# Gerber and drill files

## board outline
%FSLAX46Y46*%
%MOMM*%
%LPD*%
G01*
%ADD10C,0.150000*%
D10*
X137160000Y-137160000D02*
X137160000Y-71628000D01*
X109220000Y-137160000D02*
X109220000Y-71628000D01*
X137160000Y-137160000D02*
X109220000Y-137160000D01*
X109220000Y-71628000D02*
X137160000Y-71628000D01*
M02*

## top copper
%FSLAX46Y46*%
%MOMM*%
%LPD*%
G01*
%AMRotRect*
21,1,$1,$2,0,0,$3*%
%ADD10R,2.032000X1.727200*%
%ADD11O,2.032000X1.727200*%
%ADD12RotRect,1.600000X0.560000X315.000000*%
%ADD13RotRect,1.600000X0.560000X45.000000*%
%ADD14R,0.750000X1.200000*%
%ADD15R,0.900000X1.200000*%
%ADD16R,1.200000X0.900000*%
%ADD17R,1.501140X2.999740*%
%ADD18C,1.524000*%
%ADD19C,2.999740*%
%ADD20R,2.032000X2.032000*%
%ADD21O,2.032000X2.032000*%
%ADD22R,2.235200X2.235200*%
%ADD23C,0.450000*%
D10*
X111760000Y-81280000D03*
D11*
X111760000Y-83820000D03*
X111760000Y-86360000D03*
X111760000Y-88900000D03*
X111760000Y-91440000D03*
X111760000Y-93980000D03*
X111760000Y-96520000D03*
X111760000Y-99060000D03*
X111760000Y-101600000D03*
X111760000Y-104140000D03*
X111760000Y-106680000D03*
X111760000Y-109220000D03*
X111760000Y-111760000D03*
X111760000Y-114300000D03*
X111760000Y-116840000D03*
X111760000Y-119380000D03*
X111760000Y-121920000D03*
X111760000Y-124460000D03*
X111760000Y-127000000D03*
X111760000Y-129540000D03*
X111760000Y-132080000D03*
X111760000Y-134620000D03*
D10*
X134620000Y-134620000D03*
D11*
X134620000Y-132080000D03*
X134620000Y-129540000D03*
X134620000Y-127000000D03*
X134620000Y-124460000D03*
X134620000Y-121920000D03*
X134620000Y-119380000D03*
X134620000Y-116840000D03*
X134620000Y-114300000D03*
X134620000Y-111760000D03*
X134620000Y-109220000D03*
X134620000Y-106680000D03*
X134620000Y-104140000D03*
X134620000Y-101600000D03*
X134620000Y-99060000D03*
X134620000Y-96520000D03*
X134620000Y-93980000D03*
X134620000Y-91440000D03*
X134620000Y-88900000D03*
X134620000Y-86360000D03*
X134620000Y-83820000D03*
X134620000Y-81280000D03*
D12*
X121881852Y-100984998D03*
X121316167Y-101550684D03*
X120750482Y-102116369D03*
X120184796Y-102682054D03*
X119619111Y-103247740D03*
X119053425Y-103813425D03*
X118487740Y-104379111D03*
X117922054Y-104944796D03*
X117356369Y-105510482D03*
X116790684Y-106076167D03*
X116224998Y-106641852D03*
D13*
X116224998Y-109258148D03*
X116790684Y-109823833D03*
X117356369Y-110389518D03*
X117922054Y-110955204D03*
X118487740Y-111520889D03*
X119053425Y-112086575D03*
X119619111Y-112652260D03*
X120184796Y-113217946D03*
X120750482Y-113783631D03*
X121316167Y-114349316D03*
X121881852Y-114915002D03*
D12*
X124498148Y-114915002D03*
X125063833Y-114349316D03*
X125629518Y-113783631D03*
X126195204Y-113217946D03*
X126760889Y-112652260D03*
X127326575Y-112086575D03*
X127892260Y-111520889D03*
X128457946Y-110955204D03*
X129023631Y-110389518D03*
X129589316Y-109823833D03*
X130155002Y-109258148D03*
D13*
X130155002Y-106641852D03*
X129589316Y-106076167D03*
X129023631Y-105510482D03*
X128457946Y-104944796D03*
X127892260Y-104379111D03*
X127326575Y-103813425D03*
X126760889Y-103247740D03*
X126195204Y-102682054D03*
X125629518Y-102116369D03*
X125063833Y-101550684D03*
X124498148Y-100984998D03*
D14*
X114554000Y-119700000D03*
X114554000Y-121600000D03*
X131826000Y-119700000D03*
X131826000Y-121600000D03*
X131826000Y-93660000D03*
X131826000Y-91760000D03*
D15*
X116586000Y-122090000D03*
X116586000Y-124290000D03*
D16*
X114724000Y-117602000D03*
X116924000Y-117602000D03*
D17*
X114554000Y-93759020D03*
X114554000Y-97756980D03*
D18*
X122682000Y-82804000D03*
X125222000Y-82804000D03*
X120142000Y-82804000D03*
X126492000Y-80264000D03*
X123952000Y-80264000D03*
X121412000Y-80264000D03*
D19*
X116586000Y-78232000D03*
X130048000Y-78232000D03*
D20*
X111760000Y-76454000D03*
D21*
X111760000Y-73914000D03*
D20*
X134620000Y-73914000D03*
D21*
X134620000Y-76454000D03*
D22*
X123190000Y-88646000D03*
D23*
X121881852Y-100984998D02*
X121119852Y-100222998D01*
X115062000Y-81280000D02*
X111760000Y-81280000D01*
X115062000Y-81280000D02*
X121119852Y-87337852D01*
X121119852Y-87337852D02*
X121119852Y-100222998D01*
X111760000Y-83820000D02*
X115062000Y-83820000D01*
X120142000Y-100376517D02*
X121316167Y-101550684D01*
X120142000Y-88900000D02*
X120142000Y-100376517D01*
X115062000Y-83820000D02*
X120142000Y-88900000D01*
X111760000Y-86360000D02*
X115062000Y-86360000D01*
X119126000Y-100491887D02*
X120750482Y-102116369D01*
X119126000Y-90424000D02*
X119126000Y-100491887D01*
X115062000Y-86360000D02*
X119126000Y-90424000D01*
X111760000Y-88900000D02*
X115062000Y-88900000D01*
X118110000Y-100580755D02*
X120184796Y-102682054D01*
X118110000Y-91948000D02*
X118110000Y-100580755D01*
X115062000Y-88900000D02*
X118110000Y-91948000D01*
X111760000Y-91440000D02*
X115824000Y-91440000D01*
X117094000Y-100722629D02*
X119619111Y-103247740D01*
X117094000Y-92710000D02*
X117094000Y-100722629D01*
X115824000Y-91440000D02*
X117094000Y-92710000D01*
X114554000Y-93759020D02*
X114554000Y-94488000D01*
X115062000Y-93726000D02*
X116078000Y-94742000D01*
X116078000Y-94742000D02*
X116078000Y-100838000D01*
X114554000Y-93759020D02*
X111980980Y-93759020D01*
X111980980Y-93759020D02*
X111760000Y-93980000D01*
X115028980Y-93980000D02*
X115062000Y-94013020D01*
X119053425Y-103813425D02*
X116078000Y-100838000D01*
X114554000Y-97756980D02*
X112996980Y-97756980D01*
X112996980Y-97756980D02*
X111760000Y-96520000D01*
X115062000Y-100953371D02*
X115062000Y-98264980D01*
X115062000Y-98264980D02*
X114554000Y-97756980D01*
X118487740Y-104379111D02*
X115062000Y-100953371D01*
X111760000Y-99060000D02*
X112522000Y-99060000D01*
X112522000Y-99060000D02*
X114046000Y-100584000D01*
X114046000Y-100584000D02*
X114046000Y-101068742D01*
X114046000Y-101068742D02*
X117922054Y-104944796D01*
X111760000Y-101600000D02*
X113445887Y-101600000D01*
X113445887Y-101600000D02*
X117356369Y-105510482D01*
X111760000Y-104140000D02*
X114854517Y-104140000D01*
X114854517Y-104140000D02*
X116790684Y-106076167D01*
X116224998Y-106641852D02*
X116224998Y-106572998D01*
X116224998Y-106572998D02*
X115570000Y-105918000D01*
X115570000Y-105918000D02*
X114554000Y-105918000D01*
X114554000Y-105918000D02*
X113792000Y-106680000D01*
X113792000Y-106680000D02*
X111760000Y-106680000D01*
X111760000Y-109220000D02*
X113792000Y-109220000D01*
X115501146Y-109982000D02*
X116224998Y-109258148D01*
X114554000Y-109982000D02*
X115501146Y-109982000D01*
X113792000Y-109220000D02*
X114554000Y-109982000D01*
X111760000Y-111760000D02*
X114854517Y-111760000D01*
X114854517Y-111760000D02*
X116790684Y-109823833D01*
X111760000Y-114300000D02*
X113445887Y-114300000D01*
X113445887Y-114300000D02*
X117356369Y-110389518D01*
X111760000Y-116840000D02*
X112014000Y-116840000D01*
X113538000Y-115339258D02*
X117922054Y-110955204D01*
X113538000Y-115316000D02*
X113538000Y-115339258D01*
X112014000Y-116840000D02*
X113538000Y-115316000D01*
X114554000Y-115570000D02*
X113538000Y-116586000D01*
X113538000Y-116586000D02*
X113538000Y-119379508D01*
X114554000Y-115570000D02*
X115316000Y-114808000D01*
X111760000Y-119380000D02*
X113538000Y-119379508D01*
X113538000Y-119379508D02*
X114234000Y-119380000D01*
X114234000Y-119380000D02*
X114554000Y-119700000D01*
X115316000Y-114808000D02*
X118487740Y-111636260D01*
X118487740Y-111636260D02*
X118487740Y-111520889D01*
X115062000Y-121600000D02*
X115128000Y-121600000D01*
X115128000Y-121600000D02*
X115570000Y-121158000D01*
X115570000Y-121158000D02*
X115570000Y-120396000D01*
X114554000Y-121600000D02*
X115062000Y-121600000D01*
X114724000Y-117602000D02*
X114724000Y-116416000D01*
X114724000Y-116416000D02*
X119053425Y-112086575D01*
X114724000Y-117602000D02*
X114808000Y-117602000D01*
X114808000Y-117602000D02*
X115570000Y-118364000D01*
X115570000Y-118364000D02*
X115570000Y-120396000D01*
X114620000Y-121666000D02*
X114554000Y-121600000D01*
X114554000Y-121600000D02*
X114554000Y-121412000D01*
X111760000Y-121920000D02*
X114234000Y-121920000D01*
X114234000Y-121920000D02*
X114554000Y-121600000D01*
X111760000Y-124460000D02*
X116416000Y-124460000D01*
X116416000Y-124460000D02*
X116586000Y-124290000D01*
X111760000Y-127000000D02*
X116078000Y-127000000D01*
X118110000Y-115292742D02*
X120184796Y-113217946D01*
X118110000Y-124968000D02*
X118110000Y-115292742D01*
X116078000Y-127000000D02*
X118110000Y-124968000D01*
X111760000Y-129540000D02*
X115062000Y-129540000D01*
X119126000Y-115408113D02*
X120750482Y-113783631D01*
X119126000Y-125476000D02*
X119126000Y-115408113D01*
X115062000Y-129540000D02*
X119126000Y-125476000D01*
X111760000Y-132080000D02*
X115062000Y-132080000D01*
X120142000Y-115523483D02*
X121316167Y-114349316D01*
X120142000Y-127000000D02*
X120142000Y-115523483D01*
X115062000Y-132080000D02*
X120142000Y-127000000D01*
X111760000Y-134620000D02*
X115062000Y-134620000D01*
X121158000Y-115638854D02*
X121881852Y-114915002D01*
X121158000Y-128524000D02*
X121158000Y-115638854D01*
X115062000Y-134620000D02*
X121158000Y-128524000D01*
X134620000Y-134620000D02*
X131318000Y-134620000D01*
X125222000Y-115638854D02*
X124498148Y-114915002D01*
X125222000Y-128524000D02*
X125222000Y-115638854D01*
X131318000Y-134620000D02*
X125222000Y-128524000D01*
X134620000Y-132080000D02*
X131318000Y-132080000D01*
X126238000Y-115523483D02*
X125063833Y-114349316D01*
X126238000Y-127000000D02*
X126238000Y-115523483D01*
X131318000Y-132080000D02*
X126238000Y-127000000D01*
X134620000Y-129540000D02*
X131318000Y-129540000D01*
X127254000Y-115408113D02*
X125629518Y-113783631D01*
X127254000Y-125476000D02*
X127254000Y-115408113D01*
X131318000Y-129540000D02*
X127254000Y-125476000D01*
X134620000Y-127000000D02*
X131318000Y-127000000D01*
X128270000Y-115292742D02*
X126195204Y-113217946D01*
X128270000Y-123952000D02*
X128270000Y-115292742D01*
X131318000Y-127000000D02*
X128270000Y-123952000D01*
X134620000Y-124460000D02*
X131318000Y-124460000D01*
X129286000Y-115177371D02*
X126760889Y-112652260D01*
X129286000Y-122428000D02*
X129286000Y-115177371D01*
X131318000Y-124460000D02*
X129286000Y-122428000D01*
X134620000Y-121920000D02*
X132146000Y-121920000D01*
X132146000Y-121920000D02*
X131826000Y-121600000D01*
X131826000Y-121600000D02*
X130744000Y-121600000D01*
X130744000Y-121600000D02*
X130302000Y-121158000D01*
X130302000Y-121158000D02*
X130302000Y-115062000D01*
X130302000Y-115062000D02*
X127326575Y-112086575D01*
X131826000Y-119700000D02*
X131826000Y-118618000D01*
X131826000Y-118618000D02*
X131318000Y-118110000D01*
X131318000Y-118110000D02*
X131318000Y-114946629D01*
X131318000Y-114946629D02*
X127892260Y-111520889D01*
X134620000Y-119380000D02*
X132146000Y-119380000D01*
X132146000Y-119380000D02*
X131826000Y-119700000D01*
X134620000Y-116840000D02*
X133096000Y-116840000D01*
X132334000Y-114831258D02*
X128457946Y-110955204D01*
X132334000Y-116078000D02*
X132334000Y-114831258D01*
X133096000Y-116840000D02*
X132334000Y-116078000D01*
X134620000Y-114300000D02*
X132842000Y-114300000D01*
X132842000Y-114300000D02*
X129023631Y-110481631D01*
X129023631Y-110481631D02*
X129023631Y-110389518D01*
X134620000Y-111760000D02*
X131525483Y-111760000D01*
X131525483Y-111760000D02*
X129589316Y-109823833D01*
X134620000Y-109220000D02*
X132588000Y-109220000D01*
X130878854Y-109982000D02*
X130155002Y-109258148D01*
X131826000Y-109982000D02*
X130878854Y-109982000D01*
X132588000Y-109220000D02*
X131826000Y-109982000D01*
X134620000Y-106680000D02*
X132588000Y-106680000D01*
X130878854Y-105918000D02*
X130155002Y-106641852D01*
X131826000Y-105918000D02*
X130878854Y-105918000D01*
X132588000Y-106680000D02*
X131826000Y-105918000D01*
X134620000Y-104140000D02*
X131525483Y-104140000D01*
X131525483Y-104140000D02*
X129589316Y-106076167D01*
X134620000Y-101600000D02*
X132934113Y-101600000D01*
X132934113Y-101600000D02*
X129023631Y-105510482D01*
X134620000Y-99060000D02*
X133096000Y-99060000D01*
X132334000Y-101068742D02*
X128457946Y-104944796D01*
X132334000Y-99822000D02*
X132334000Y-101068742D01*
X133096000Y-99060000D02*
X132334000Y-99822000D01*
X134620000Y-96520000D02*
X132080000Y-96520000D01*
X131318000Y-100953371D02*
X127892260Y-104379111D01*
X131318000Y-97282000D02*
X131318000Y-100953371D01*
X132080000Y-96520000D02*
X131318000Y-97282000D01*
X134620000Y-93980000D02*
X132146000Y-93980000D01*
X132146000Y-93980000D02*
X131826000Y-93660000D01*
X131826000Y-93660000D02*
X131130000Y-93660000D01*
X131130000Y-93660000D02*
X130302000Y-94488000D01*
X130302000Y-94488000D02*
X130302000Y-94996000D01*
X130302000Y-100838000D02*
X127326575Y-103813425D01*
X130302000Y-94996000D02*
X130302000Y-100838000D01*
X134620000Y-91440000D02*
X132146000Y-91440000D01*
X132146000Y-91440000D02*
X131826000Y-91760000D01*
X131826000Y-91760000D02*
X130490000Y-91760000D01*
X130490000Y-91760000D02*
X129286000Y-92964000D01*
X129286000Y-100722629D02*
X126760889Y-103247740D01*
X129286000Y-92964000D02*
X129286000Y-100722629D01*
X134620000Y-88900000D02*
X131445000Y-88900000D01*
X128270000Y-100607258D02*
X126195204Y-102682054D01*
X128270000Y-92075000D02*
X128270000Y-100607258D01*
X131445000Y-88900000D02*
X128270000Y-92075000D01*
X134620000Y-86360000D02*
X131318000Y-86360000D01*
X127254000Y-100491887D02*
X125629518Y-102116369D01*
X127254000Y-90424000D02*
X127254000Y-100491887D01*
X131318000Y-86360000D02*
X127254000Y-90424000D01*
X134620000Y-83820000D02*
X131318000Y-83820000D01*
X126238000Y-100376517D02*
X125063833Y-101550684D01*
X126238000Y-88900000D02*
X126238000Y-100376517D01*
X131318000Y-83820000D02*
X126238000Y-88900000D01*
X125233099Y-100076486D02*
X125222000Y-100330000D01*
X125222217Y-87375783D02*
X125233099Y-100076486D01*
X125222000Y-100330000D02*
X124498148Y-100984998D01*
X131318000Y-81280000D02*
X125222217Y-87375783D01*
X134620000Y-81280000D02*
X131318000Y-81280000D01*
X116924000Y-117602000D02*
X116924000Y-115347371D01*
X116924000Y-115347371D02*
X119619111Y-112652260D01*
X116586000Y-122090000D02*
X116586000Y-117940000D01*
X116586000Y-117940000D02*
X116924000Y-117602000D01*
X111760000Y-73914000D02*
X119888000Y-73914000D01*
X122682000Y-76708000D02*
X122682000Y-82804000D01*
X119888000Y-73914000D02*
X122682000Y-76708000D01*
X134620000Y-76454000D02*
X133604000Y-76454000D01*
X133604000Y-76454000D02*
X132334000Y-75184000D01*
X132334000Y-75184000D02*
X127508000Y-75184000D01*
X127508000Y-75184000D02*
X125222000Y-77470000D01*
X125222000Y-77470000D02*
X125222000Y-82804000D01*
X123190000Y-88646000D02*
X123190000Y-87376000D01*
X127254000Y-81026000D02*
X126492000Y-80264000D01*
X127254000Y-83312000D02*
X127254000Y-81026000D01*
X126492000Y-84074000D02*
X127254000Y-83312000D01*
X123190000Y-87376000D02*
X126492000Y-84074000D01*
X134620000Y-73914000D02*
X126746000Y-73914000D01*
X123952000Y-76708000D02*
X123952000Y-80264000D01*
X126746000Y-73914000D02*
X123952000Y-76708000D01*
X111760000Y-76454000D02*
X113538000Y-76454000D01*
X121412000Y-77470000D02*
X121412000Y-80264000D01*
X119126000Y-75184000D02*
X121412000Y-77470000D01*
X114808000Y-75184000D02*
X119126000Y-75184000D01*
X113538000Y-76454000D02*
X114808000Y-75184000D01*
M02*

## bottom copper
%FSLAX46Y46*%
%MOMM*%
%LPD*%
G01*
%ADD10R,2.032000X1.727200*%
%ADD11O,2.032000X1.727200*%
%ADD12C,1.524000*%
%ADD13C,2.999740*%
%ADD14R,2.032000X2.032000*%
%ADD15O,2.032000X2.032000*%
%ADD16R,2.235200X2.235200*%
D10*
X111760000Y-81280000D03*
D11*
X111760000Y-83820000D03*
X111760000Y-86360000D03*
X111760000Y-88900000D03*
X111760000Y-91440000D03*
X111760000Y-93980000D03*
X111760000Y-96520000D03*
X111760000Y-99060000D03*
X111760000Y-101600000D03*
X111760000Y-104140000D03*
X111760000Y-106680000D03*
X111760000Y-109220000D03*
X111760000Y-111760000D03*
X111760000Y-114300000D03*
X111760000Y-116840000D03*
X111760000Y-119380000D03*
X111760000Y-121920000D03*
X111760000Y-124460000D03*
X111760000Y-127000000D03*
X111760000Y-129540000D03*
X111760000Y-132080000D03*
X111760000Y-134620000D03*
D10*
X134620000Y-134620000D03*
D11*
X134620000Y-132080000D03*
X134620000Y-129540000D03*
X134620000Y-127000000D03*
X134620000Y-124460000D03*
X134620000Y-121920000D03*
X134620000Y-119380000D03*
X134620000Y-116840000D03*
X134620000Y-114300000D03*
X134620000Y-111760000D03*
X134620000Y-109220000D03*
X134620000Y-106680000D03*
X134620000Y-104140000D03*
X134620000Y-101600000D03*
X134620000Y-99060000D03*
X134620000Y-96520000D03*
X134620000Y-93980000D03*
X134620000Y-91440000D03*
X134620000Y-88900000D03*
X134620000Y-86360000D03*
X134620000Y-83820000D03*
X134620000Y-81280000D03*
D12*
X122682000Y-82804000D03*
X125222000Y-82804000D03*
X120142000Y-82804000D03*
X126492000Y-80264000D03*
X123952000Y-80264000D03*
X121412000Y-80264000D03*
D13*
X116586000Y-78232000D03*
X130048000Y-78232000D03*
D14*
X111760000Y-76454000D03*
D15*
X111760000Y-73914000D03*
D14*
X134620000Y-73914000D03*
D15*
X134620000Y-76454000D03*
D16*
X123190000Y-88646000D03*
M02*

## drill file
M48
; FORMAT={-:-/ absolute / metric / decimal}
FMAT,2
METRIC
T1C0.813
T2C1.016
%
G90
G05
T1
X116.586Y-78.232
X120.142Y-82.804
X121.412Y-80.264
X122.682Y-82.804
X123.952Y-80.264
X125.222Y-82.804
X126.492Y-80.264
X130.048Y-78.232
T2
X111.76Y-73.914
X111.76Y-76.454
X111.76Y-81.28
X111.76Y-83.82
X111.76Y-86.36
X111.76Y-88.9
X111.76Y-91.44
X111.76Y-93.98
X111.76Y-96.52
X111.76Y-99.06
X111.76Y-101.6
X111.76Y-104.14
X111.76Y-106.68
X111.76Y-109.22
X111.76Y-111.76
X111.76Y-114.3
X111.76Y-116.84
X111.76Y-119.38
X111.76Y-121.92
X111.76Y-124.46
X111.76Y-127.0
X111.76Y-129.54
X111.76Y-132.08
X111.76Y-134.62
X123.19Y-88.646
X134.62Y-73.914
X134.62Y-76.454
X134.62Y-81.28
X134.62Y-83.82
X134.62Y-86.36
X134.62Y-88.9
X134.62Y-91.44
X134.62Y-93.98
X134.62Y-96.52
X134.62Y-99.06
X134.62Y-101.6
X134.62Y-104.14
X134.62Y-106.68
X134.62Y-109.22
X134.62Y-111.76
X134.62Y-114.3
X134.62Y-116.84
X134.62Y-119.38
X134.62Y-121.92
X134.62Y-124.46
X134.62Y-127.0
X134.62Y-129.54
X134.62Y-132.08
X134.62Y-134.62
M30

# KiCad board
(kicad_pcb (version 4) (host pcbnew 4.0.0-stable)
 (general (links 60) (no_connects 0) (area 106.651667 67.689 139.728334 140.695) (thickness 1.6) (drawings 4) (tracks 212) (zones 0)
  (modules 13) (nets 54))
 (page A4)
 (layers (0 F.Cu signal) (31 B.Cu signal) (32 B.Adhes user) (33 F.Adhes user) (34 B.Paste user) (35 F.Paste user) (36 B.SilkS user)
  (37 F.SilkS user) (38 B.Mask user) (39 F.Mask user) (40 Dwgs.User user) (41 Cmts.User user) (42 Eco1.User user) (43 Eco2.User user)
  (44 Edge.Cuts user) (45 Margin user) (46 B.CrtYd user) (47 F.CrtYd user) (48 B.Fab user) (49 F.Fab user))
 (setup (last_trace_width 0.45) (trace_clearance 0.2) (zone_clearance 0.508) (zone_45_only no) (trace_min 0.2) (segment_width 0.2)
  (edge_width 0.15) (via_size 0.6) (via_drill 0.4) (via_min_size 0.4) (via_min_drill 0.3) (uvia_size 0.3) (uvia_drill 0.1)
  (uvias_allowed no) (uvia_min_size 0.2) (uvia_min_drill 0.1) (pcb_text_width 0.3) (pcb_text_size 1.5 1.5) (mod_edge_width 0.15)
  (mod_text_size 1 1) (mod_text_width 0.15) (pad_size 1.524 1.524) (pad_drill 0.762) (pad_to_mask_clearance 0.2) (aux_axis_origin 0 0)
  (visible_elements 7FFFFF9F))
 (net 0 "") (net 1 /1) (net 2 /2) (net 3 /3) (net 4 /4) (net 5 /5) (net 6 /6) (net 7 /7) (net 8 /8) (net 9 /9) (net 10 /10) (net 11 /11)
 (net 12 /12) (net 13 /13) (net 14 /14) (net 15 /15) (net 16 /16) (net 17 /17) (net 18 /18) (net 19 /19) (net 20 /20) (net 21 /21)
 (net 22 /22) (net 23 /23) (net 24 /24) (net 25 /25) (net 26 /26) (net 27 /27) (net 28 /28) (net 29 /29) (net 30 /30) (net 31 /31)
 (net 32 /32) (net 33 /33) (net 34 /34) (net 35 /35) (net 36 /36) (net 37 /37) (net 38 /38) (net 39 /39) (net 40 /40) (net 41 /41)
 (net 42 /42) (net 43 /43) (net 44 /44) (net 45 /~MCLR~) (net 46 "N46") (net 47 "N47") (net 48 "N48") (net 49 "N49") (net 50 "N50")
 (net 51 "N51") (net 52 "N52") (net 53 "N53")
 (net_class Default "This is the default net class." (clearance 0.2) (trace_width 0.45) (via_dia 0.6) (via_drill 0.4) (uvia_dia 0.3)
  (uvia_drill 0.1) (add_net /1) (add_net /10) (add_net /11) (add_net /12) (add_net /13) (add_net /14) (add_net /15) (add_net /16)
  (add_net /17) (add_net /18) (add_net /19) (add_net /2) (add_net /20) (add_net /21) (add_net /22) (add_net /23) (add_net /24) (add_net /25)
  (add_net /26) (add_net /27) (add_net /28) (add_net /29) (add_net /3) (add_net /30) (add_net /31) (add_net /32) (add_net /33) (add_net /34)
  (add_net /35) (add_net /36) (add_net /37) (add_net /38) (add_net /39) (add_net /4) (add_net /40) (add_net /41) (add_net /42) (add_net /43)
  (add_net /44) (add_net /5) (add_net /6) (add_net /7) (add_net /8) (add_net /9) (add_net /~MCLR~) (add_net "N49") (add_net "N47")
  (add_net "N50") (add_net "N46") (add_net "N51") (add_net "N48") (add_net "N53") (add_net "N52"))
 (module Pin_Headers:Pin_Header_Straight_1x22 (layer B.Cu) (at 111.76 81.28 180)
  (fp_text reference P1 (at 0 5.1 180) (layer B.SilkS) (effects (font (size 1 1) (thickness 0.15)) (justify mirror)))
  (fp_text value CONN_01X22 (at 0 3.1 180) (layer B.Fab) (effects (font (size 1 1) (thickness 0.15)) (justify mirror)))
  (pad 1 thru_hole rect (at 0 0 180) (size 2.032 1.7272) (drill 1.016) (layers *.Cu *.Mask B.SilkS) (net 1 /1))
  (pad 2 thru_hole oval (at 0 -2.54 180) (size 2.032 1.7272) (drill 1.016) (layers *.Cu *.Mask B.SilkS) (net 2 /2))
  (pad 3 thru_hole oval (at 0 -5.08 180) (size 2.032 1.7272) (drill 1.016) (layers *.Cu *.Mask B.SilkS) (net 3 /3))
  (pad 4 thru_hole oval (at 0 -7.62 180) (size 2.032 1.7272) (drill 1.016) (layers *.Cu *.Mask B.SilkS) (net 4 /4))
  (pad 5 thru_hole oval (at 0 -10.16 180) (size 2.032 1.7272) (drill 1.016) (layers *.Cu *.Mask B.SilkS) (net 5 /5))
  (pad 6 thru_hole oval (at 0 -12.7 180) (size 2.032 1.7272) (drill 1.016) (layers *.Cu *.Mask B.SilkS) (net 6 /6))
  (pad 7 thru_hole oval (at 0 -15.24 180) (size 2.032 1.7272) (drill 1.016) (layers *.Cu *.Mask B.SilkS) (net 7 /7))
  (pad 8 thru_hole oval (at 0 -17.78 180) (size 2.032 1.7272) (drill 1.016) (layers *.Cu *.Mask B.SilkS) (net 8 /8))
  (pad 9 thru_hole oval (at 0 -20.32 180) (size 2.032 1.7272) (drill 1.016) (layers *.Cu *.Mask B.SilkS) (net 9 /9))
  (pad 10 thru_hole oval (at 0 -22.86 180) (size 2.032 1.7272) (drill 1.016) (layers *.Cu *.Mask B.SilkS) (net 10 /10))
  (pad 11 thru_hole oval (at 0 -25.4 180) (size 2.032 1.7272) (drill 1.016) (layers *.Cu *.Mask B.SilkS) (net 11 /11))
  (pad 12 thru_hole oval (at 0 -27.94 180) (size 2.032 1.7272) (drill 1.016) (layers *.Cu *.Mask B.SilkS) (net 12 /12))
  (pad 13 thru_hole oval (at 0 -30.48 180) (size 2.032 1.7272) (drill 1.016) (layers *.Cu *.Mask B.SilkS) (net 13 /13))
  (pad 14 thru_hole oval (at 0 -33.02 180) (size 2.032 1.7272) (drill 1.016) (layers *.Cu *.Mask B.SilkS) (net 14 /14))
  (pad 15 thru_hole oval (at 0 -35.56 180) (size 2.032 1.7272) (drill 1.016) (layers *.Cu *.Mask B.SilkS) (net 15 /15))
  (pad 16 thru_hole oval (at 0 -38.1 180) (size 2.032 1.7272) (drill 1.016) (layers *.Cu *.Mask B.SilkS) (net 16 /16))
  (pad 17 thru_hole oval (at 0 -40.64 180) (size 2.032 1.7272) (drill 1.016) (layers *.Cu *.Mask B.SilkS) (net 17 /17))
  (pad 18 thru_hole oval (at 0 -43.18 180) (size 2.032 1.7272) (drill 1.016) (layers *.Cu *.Mask B.SilkS) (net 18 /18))
  (pad 19 thru_hole oval (at 0 -45.72 180) (size 2.032 1.7272) (drill 1.016) (layers *.Cu *.Mask B.SilkS) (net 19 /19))
  (pad 20 thru_hole oval (at 0 -48.26 180) (size 2.032 1.7272) (drill 1.016) (layers *.Cu *.Mask B.SilkS) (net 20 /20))
  (pad 21 thru_hole oval (at 0 -50.8 180) (size 2.032 1.7272) (drill 1.016) (layers *.Cu *.Mask B.SilkS) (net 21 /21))
  (pad 22 thru_hole oval (at 0 -53.34 180) (size 2.032 1.7272) (drill 1.016) (layers *.Cu *.Mask B.SilkS) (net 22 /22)))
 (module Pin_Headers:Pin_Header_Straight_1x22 (layer B.Cu) (at 134.62 134.62)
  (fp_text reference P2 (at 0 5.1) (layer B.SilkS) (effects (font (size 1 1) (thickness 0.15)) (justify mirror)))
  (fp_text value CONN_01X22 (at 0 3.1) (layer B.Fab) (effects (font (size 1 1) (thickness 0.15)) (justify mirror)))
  (pad 1 thru_hole rect (at 0 0) (size 2.032 1.7272) (drill 1.016) (layers *.Cu *.Mask B.SilkS) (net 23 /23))
  (pad 2 thru_hole oval (at 0 -2.54) (size 2.032 1.7272) (drill 1.016) (layers *.Cu *.Mask B.SilkS) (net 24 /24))
  (pad 3 thru_hole oval (at 0 -5.08) (size 2.032 1.7272) (drill 1.016) (layers *.Cu *.Mask B.SilkS) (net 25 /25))
  (pad 4 thru_hole oval (at 0 -7.62) (size 2.032 1.7272) (drill 1.016) (layers *.Cu *.Mask B.SilkS) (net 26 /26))
  (pad 5 thru_hole oval (at 0 -10.16) (size 2.032 1.7272) (drill 1.016) (layers *.Cu *.Mask B.SilkS) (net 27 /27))
  (pad 6 thru_hole oval (at 0 -12.7) (size 2.032 1.7272) (drill 1.016) (layers *.Cu *.Mask B.SilkS) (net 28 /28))
  (pad 7 thru_hole oval (at 0 -15.24) (size 2.032 1.7272) (drill 1.016) (layers *.Cu *.Mask B.SilkS) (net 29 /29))
  (pad 8 thru_hole oval (at 0 -17.78) (size 2.032 1.7272) (drill 1.016) (layers *.Cu *.Mask B.SilkS) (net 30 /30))
  (pad 9 thru_hole oval (at 0 -20.32) (size 2.032 1.7272) (drill 1.016) (layers *.Cu *.Mask B.SilkS) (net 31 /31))
  (pad 10 thru_hole oval (at 0 -22.86) (size 2.032 1.7272) (drill 1.016) (layers *.Cu *.Mask B.SilkS) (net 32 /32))
  (pad 11 thru_hole oval (at 0 -25.4) (size 2.032 1.7272) (drill 1.016) (layers *.Cu *.Mask B.SilkS) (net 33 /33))
  (pad 12 thru_hole oval (at 0 -27.94) (size 2.032 1.7272) (drill 1.016) (layers *.Cu *.Mask B.SilkS) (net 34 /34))
  (pad 13 thru_hole oval (at 0 -30.48) (size 2.032 1.7272) (drill 1.016) (layers *.Cu *.Mask B.SilkS) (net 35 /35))
  (pad 14 thru_hole oval (at 0 -33.02) (size 2.032 1.7272) (drill 1.016) (layers *.Cu *.Mask B.SilkS) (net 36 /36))
  (pad 15 thru_hole oval (at 0 -35.56) (size 2.032 1.7272) (drill 1.016) (layers *.Cu *.Mask B.SilkS) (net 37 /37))
  (pad 16 thru_hole oval (at 0 -38.1) (size 2.032 1.7272) (drill 1.016) (layers *.Cu *.Mask B.SilkS) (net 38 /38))
  (pad 17 thru_hole oval (at 0 -40.64) (size 2.032 1.7272) (drill 1.016) (layers *.Cu *.Mask B.SilkS) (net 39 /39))
  (pad 18 thru_hole oval (at 0 -43.18) (size 2.032 1.7272) (drill 1.016) (layers *.Cu *.Mask B.SilkS) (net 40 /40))
  (pad 19 thru_hole oval (at 0 -45.72) (size 2.032 1.7272) (drill 1.016) (layers *.Cu *.Mask B.SilkS) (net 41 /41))
  (pad 20 thru_hole oval (at 0 -48.26) (size 2.032 1.7272) (drill 1.016) (layers *.Cu *.Mask B.SilkS) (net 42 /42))
  (pad 21 thru_hole oval (at 0 -50.8) (size 2.032 1.7272) (drill 1.016) (layers *.Cu *.Mask B.SilkS) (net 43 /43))
  (pad 22 thru_hole oval (at 0 -53.34) (size 2.032 1.7272) (drill 1.016) (layers *.Cu *.Mask B.SilkS) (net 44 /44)))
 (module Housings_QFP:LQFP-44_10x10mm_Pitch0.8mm (layer F.Cu) (at 123.19 107.95 315)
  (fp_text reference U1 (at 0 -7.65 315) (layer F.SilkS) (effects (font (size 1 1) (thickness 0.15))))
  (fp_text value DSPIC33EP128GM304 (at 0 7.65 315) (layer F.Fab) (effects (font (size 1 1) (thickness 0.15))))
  (pad 1 smd rect (at -5.85 -4 315) (size 1.6 0.56) (layers F.Cu F.Paste F.Mask) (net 1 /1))
  (pad 2 smd rect (at -5.85 -3.2 315) (size 1.6 0.56) (layers F.Cu F.Paste F.Mask) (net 2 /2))
  (pad 3 smd rect (at -5.85 -2.4 315) (size 1.6 0.56) (layers F.Cu F.Paste F.Mask) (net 3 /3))
  (pad 4 smd rect (at -5.85 -1.6 315) (size 1.6 0.56) (layers F.Cu F.Paste F.Mask) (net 4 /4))
  (pad 5 smd rect (at -5.85 -0.8 315) (size 1.6 0.56) (layers F.Cu F.Paste F.Mask) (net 5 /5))
  (pad 6 smd rect (at -5.85 0 315) (size 1.6 0.56) (layers F.Cu F.Paste F.Mask) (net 6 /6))
  (pad 7 smd rect (at -5.85 0.8 315) (size 1.6 0.56) (layers F.Cu F.Paste F.Mask) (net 7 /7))
  (pad 8 smd rect (at -5.85 1.6 315) (size 1.6 0.56) (layers F.Cu F.Paste F.Mask) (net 8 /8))
  (pad 9 smd rect (at -5.85 2.4 315) (size 1.6 0.56) (layers F.Cu F.Paste F.Mask) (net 9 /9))
  (pad 10 smd rect (at -5.85 3.2 315) (size 1.6 0.56) (layers F.Cu F.Paste F.Mask) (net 10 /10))
  (pad 11 smd rect (at -5.85 4 315) (size 1.6 0.56) (layers F.Cu F.Paste F.Mask) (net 11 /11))
  (pad 12 smd rect (at -4 5.85 45) (size 1.6 0.56) (layers F.Cu F.Paste F.Mask) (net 12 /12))
  (pad 13 smd rect (at -3.2 5.85 45) (size 1.6 0.56) (layers F.Cu F.Paste F.Mask) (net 13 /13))
  (pad 14 smd rect (at -2.4 5.85 45) (size 1.6 0.56) (layers F.Cu F.Paste F.Mask) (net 14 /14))
  (pad 15 smd rect (at -1.6 5.85 45) (size 1.6 0.56) (layers F.Cu F.Paste F.Mask) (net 15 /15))
  (pad 16 smd rect (at -0.8 5.85 45) (size 1.6 0.56) (layers F.Cu F.Paste F.Mask) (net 16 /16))
  (pad 17 smd rect (at 0 5.85 45) (size 1.6 0.56) (layers F.Cu F.Paste F.Mask) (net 17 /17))
  (pad 18 smd rect (at 0.8 5.85 45) (size 1.6 0.56) (layers F.Cu F.Paste F.Mask) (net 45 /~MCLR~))
  (pad 19 smd rect (at 1.6 5.85 45) (size 1.6 0.56) (layers F.Cu F.Paste F.Mask) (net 19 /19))
  (pad 20 smd rect (at 2.4 5.85 45) (size 1.6 0.56) (layers F.Cu F.Paste F.Mask) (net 20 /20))
  (pad 21 smd rect (at 3.2 5.85 45) (size 1.6 0.56) (layers F.Cu F.Paste F.Mask) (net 21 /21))
  (pad 22 smd rect (at 4 5.85 45) (size 1.6 0.56) (layers F.Cu F.Paste F.Mask) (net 22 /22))
  (pad 23 smd rect (at 5.85 4 315) (size 1.6 0.56) (layers F.Cu F.Paste F.Mask) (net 23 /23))
  (pad 24 smd rect (at 5.85 3.2 315) (size 1.6 0.56) (layers F.Cu F.Paste F.Mask) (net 24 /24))
  (pad 25 smd rect (at 5.85 2.4 315) (size 1.6 0.56) (layers F.Cu F.Paste F.Mask) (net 25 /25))
  (pad 26 smd rect (at 5.85 1.6 315) (size 1.6 0.56) (layers F.Cu F.Paste F.Mask) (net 26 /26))
  (pad 27 smd rect (at 5.85 0.8 315) (size 1.6 0.56) (layers F.Cu F.Paste F.Mask) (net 27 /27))
  (pad 28 smd rect (at 5.85 0 315) (size 1.6 0.56) (layers F.Cu F.Paste F.Mask) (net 28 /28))
  (pad 29 smd rect (at 5.85 -0.8 315) (size 1.6 0.56) (layers F.Cu F.Paste F.Mask) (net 29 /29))
  (pad 30 smd rect (at 5.85 -1.6 315) (size 1.6 0.56) (layers F.Cu F.Paste F.Mask) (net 30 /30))
  (pad 31 smd rect (at 5.85 -2.4 315) (size 1.6 0.56) (layers F.Cu F.Paste F.Mask) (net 31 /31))
  (pad 32 smd rect (at 5.85 -3.2 315) (size 1.6 0.56) (layers F.Cu F.Paste F.Mask) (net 32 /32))
  (pad 33 smd rect (at 5.85 -4 315) (size 1.6 0.56) (layers F.Cu F.Paste F.Mask) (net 33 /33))
  (pad 34 smd rect (at 4 -5.85 45) (size 1.6 0.56) (layers F.Cu F.Paste F.Mask) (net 34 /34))
  (pad 35 smd rect (at 3.2 -5.85 45) (size 1.6 0.56) (layers F.Cu F.Paste F.Mask) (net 35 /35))
  (pad 36 smd rect (at 2.4 -5.85 45) (size 1.6 0.56) (layers F.Cu F.Paste F.Mask) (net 36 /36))
  (pad 37 smd rect (at 1.6 -5.85 45) (size 1.6 0.56) (layers F.Cu F.Paste F.Mask) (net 37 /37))
  (pad 38 smd rect (at 0.8 -5.85 45) (size 1.6 0.56) (layers F.Cu F.Paste F.Mask) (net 38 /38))
  (pad 39 smd rect (at 0 -5.85 45) (size 1.6 0.56) (layers F.Cu F.Paste F.Mask) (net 39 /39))
  (pad 40 smd rect (at -0.8 -5.85 45) (size 1.6 0.56) (layers F.Cu F.Paste F.Mask) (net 40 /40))
  (pad 41 smd rect (at -1.6 -5.85 45) (size 1.6 0.56) (layers F.Cu F.Paste F.Mask) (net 41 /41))
  (pad 42 smd rect (at -2.4 -5.85 45) (size 1.6 0.56) (layers F.Cu F.Paste F.Mask) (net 42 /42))
  (pad 43 smd rect (at -3.2 -5.85 45) (size 1.6 0.56) (layers F.Cu F.Paste F.Mask) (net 43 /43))
  (pad 44 smd rect (at -4 -5.85 45) (size 1.6 0.56) (layers F.Cu F.Paste F.Mask) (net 44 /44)))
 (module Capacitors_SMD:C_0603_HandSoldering (layer F.Cu) (at 114.554 120.65 270)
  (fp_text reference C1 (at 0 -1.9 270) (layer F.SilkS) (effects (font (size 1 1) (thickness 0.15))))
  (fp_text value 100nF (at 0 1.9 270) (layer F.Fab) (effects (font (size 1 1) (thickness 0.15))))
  (pad 1 smd rect (at -0.95 0 270) (size 1.2 0.75) (layers F.Cu F.Paste F.Mask) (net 16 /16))
  (pad 2 smd rect (at 0.95 0 270) (size 1.2 0.75) (layers F.Cu F.Paste F.Mask) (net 17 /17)))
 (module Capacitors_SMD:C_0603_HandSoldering (layer F.Cu) (at 131.826 120.65 270)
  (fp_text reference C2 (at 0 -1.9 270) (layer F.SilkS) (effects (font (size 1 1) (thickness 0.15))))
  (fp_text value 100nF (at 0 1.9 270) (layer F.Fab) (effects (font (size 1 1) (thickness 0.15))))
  (pad 1 smd rect (at -0.95 0 270) (size 1.2 0.75) (layers F.Cu F.Paste F.Mask) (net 29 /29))
  (pad 2 smd rect (at 0.95 0 270) (size 1.2 0.75) (layers F.Cu F.Paste F.Mask) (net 28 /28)))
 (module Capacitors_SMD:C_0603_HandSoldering (layer F.Cu) (at 131.826 92.71 90)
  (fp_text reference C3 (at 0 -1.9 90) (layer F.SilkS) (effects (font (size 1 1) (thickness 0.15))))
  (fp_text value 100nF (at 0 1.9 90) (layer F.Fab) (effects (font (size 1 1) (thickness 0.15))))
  (pad 1 smd rect (at -0.95 0 90) (size 1.2 0.75) (layers F.Cu F.Paste F.Mask) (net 39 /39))
  (pad 2 smd rect (at 0.95 0 90) (size 1.2 0.75) (layers F.Cu F.Paste F.Mask) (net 40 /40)))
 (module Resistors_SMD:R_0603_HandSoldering (layer F.Cu) (at 116.586 123.19 270)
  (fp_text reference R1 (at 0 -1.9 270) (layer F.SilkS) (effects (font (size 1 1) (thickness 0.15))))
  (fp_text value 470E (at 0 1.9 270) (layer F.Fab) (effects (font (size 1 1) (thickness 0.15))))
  (pad 1 smd rect (at -1.1 0 270) (size 1.2 0.9) (layers F.Cu F.Paste F.Mask) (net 45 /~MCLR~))
  (pad 2 smd rect (at 1.1 0 270) (size 1.2 0.9) (layers F.Cu F.Paste F.Mask) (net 18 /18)))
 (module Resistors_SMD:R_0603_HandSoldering (layer F.Cu) (at 115.824 117.602)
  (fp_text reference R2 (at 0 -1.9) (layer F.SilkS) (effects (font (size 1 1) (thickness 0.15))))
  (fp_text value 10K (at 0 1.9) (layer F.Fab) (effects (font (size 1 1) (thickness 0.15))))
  (pad 1 smd rect (at -1.1 0) (size 1.2 0.9) (layers F.Cu F.Paste F.Mask) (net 17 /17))
  (pad 2 smd rect (at 1.1 0) (size 1.2 0.9) (layers F.Cu F.Paste F.Mask) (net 45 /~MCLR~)))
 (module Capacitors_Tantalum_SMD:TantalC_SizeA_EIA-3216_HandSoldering (layer F.Cu) (at 114.554 95.758 90)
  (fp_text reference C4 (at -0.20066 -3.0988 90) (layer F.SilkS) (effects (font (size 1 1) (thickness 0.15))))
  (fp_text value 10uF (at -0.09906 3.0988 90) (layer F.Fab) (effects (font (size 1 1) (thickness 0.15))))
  (pad 2 smd rect (at 1.99898 0 90) (size 2.99974 1.50114) (layers F.Cu F.Paste F.Mask) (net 6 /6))
  (pad 1 smd rect (at -1.99898 0 90) (size 2.99974 1.50114) (layers F.Cu F.Paste F.Mask) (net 7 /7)))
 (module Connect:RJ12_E (layer F.Cu) (at 123.19 73.914 180)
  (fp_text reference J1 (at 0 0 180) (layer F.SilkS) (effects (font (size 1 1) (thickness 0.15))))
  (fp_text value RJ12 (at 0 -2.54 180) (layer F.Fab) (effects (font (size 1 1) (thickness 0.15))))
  (pad 4 thru_hole circle (at 0.508 -8.89 180) (size 1.524 1.524) (drill 0.8128) (layers *.Cu *.Mask F.SilkS) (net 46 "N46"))
  (pad 2 thru_hole circle (at -2.032 -8.89 180) (size 1.524 1.524) (drill 0.8128) (layers *.Cu *.Mask F.SilkS) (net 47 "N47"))
  (pad 6 thru_hole circle (at 3.048 -8.89 180) (size 1.524 1.524) (drill 0.8128) (layers *.Cu *.Mask F.SilkS) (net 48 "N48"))
  (pad 1 thru_hole circle (at -3.302 -6.35 180) (size 1.524 1.524) (drill 0.8128) (layers *.Cu *.Mask F.SilkS) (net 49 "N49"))
  (pad 3 thru_hole circle (at -0.762 -6.35 180) (size 1.524 1.524) (drill 0.8128) (layers *.Cu *.Mask F.SilkS) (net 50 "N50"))
  (pad 5 thru_hole circle (at 1.778 -6.35 180) (size 1.524 1.524) (drill 0.8128) (layers *.Cu *.Mask F.SilkS) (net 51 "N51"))
  (pad 8 thru_hole circle (at 6.604 -4.318 180) (size 2.99974 2.99974) (drill 0.8128) (layers *.Cu *.Mask F.SilkS) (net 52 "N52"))
  (pad 7 thru_hole circle (at -6.858 -4.318 180) (size 2.99974 2.99974) (drill 0.8128) (layers *.Cu *.Mask F.SilkS) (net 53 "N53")))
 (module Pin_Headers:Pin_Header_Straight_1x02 (layer F.Cu) (at 111.76 76.454 180)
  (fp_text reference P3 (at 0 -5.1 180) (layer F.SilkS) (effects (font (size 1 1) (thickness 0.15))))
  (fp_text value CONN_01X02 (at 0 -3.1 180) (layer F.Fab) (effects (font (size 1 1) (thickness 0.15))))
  (pad 1 thru_hole rect (at 0 0 180) (size 2.032 2.032) (drill 1.016) (layers *.Cu *.Mask F.SilkS) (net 51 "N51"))
  (pad 2 thru_hole oval (at 0 2.54 180) (size 2.032 2.032) (drill 1.016) (layers *.Cu *.Mask F.SilkS) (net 46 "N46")))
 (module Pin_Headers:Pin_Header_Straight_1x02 (layer F.Cu) (at 134.62 73.914)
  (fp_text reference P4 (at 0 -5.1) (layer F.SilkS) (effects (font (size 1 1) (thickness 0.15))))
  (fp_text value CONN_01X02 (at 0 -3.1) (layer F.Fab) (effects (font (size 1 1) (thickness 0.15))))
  (pad 1 thru_hole rect (at 0 0) (size 2.032 2.032) (drill 1.016) (layers *.Cu *.Mask F.SilkS) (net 50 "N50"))
  (pad 2 thru_hole oval (at 0 2.54) (size 2.032 2.032) (drill 1.016) (layers *.Cu *.Mask F.SilkS) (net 47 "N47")))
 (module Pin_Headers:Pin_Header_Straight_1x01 (layer F.Cu) (at 123.19 88.646)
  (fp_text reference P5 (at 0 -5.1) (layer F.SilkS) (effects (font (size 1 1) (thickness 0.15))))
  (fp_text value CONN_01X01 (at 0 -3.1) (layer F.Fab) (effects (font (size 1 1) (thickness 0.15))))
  (pad 1 thru_hole rect (at 0 0) (size 2.2352 2.2352) (drill 1.016) (layers *.Cu *.Mask F.SilkS) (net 49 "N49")))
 (gr_line (start 137.16 137.16) (end 137.16 71.628) (angle 90) (layer Edge.Cuts) (width 0.15))
 (gr_line (start 109.22 137.16) (end 109.22 71.628) (angle 90) (layer Edge.Cuts) (width 0.15))
 (gr_line (start 137.16 137.16) (end 109.22 137.16) (angle 90) (layer Edge.Cuts) (width 0.15))
 (gr_line (start 109.22 71.628) (end 137.16 71.628) (angle 90) (layer Edge.Cuts) (width 0.15))
 (segment (start 121.881852 100.984998) (end 121.119852 100.222998) (width 0.45) (layer F.Cu) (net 1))
 (segment (start 115.062 81.28) (end 111.76 81.28) (width 0.45) (layer F.Cu) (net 1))
 (segment (start 115.062 81.28) (end 121.119852 87.337852) (width 0.45) (layer F.Cu) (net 1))
 (segment (start 121.119852 87.337852) (end 121.119852 100.222998) (width 0.45) (layer F.Cu) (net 1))
 (segment (start 111.76 83.82) (end 115.062 83.82) (width 0.45) (layer F.Cu) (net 2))
 (segment (start 120.142 100.376517) (end 121.316167 101.550684) (width 0.45) (layer F.Cu) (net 2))
 (segment (start 120.142 88.9) (end 120.142 100.376517) (width 0.45) (layer F.Cu) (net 2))
 (segment (start 115.062 83.82) (end 120.142 88.9) (width 0.45) (layer F.Cu) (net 2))
 (segment (start 111.76 86.36) (end 115.062 86.36) (width 0.45) (layer F.Cu) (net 3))
 (segment (start 119.126 100.491887) (end 120.750482 102.116369) (width 0.45) (layer F.Cu) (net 3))
 (segment (start 119.126 90.424) (end 119.126 100.491887) (width 0.45) (layer F.Cu) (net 3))
 (segment (start 115.062 86.36) (end 119.126 90.424) (width 0.45) (layer F.Cu) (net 3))
 (segment (start 111.76 88.9) (end 115.062 88.9) (width 0.45) (layer F.Cu) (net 4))
 (segment (start 118.11 100.580755) (end 120.184796 102.682054) (width 0.45) (layer F.Cu) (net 4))
 (segment (start 118.11 91.948) (end 118.11 100.580755) (width 0.45) (layer F.Cu) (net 4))
 (segment (start 115.062 88.9) (end 118.11 91.948) (width 0.45) (layer F.Cu) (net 4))
 (segment (start 111.76 91.44) (end 115.824 91.44) (width 0.45) (layer F.Cu) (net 5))
 (segment (start 117.094 100.722629) (end 119.619111 103.24774) (width 0.45) (layer F.Cu) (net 5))
 (segment (start 117.094 92.71) (end 117.094 100.722629) (width 0.45) (layer F.Cu) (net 5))
 (segment (start 115.824 91.44) (end 117.094 92.71) (width 0.45) (layer F.Cu) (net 5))
 (segment (start 114.554 93.75902) (end 114.554 94.488) (width 0.45) (layer F.Cu) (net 6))
 (segment (start 115.062 93.726) (end 116.078 94.742) (width 0.45) (layer F.Cu) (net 6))
 (segment (start 116.078 94.742) (end 116.078 100.838) (width 0.45) (layer F.Cu) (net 6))
 (segment (start 114.554 93.75902) (end 111.98098 93.75902) (width 0.45) (layer F.Cu) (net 6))
 (segment (start 111.98098 93.75902) (end 111.76 93.98) (width 0.45) (layer F.Cu) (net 6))
 (segment (start 115.02898 93.98) (end 115.062 94.01302) (width 0.45) (layer F.Cu) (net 6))
 (segment (start 119.053425 103.813425) (end 116.078 100.838) (width 0.45) (layer F.Cu) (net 6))
 (segment (start 114.554 97.75698) (end 112.99698 97.75698) (width 0.45) (layer F.Cu) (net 7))
 (segment (start 112.99698 97.75698) (end 111.76 96.52) (width 0.45) (layer F.Cu) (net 7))
 (segment (start 115.062 100.953371) (end 115.062 98.26498) (width 0.45) (layer F.Cu) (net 7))
 (segment (start 115.062 98.26498) (end 114.554 97.75698) (width 0.45) (layer F.Cu) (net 7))
 (segment (start 118.48774 104.379111) (end 115.062 100.953371) (width 0.45) (layer F.Cu) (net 7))
 (segment (start 111.76 99.06) (end 112.522 99.06) (width 0.45) (layer F.Cu) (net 8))
 (segment (start 112.522 99.06) (end 114.046 100.584) (width 0.45) (layer F.Cu) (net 8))
 (segment (start 114.046 100.584) (end 114.046 101.068742) (width 0.45) (layer F.Cu) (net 8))
 (segment (start 114.046 101.068742) (end 117.922054 104.944796) (width 0.45) (layer F.Cu) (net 8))
 (segment (start 111.76 101.6) (end 113.445887 101.6) (width 0.45) (layer F.Cu) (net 9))
 (segment (start 113.445887 101.6) (end 117.356369 105.510482) (width 0.45) (layer F.Cu) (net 9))
 (segment (start 111.76 104.14) (end 114.854517 104.14) (width 0.45) (layer F.Cu) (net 10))
 (segment (start 114.854517 104.14) (end 116.790684 106.076167) (width 0.45) (layer F.Cu) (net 10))
 (segment (start 116.224998 106.641852) (end 116.224998 106.572998) (width 0.45) (layer F.Cu) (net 11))
 (segment (start 116.224998 106.572998) (end 115.57 105.918) (width 0.45) (layer F.Cu) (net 11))
 (segment (start 115.57 105.918) (end 114.554 105.918) (width 0.45) (layer F.Cu) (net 11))
 (segment (start 114.554 105.918) (end 113.792 106.68) (width 0.45) (layer F.Cu) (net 11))
 (segment (start 113.792 106.68) (end 111.76 106.68) (width 0.45) (layer F.Cu) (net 11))
 (segment (start 111.76 109.22) (end 113.792 109.22) (width 0.45) (layer F.Cu) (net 12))
 (segment (start 115.501146 109.982) (end 116.224998 109.258148) (width 0.45) (layer F.Cu) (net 12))
 (segment (start 114.554 109.982) (end 115.501146 109.982) (width 0.45) (layer F.Cu) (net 12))
 (segment (start 113.792 109.22) (end 114.554 109.982) (width 0.45) (layer F.Cu) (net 12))
 (segment (start 111.76 111.76) (end 114.854517 111.76) (width 0.45) (layer F.Cu) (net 13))
 (segment (start 114.854517 111.76) (end 116.790684 109.823833) (width 0.45) (layer F.Cu) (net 13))
 (segment (start 111.76 114.3) (end 113.445887 114.3) (width 0.45) (layer F.Cu) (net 14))
 (segment (start 113.445887 114.3) (end 117.356369 110.389518) (width 0.45) (layer F.Cu) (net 14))
 (segment (start 111.76 116.84) (end 112.014 116.84) (width 0.45) (layer F.Cu) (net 15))
 (segment (start 113.538 115.339258) (end 117.922054 110.955204) (width 0.45) (layer F.Cu) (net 15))
 (segment (start 113.538 115.316) (end 113.538 115.339258) (width 0.45) (layer F.Cu) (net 15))
 (segment (start 112.014 116.84) (end 113.538 115.316) (width 0.45) (layer F.Cu) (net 15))
 (segment (start 114.554 115.57) (end 113.538 116.586) (width 0.45) (layer F.Cu) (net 16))
 (segment (start 113.538 116.586) (end 113.538 119.379508) (width 0.45) (layer F.Cu) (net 16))
 (segment (start 114.554 115.57) (end 115.316 114.808) (width 0.45) (layer F.Cu) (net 16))
 (segment (start 111.76 119.38) (end 113.538 119.379508) (width 0.45) (layer F.Cu) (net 16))
 (segment (start 113.538 119.379508) (end 114.234 119.38) (width 0.45) (layer F.Cu) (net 16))
 (segment (start 114.234 119.38) (end 114.554 119.7) (width 0.45) (layer F.Cu) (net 16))
 (segment (start 115.316 114.808) (end 118.48774 111.63626) (width 0.45) (layer F.Cu) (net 16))
 (segment (start 118.48774 111.63626) (end 118.48774 111.520889) (width 0.45) (layer F.Cu) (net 16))
 (segment (start 115.062 121.6) (end 115.128 121.6) (width 0.45) (layer F.Cu) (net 17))
 (segment (start 115.128 121.6) (end 115.57 121.158) (width 0.45) (layer F.Cu) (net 17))
 (segment (start 115.57 121.158) (end 115.57 120.396) (width 0.45) (layer F.Cu) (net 17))
 (segment (start 114.554 121.6) (end 115.062 121.6) (width 0.45) (layer F.Cu) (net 17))
 (segment (start 114.724 117.602) (end 114.724 116.416) (width 0.45) (layer F.Cu) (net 17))
 (segment (start 114.724 116.416) (end 119.053425 112.086575) (width 0.45) (layer F.Cu) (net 17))
 (segment (start 114.724 117.602) (end 114.808 117.602) (width 0.45) (layer F.Cu) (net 17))
 (segment (start 114.808 117.602) (end 115.57 118.364) (width 0.45) (layer F.Cu) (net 17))
 (segment (start 115.57 118.364) (end 115.57 120.396) (width 0.45) (layer F.Cu) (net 17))
 (segment (start 114.62 121.666) (end 114.554 121.6) (width 0.45) (layer F.Cu) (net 17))
 (segment (start 114.554 121.6) (end 114.554 121.412) (width 0.45) (layer F.Cu) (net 17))
 (segment (start 111.76 121.92) (end 114.234 121.92) (width 0.45) (layer F.Cu) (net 17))
 (segment (start 114.234 121.92) (end 114.554 121.6) (width 0.45) (layer F.Cu) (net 17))
 (segment (start 111.76 124.46) (end 116.416 124.46) (width 0.45) (layer F.Cu) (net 18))
 (segment (start 116.416 124.46) (end 116.586 124.29) (width 0.45) (layer F.Cu) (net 18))
 (segment (start 111.76 127) (end 116.078 127) (width 0.45) (layer F.Cu) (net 19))
 (segment (start 118.11 115.292742) (end 120.184796 113.217946) (width 0.45) (layer F.Cu) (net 19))
 (segment (start 118.11 124.968) (end 118.11 115.292742) (width 0.45) (layer F.Cu) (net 19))
 (segment (start 116.078 127) (end 118.11 124.968) (width 0.45) (layer F.Cu) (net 19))
 (segment (start 111.76 129.54) (end 115.062 129.54) (width 0.45) (layer F.Cu) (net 20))
 (segment (start 119.126 115.408113) (end 120.750482 113.783631) (width 0.45) (layer F.Cu) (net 20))
 (segment (start 119.126 125.476) (end 119.126 115.408113) (width 0.45) (layer F.Cu) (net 20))
 (segment (start 115.062 129.54) (end 119.126 125.476) (width 0.45) (layer F.Cu) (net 20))
 (segment (start 111.76 132.08) (end 115.062 132.08) (width 0.45) (layer F.Cu) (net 21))
 (segment (start 120.142 115.523483) (end 121.316167 114.349316) (width 0.45) (layer F.Cu) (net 21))
 (segment (start 120.142 127) (end 120.142 115.523483) (width 0.45) (layer F.Cu) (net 21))
 (segment (start 115.062 132.08) (end 120.142 127) (width 0.45) (layer F.Cu) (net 21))
 (segment (start 111.76 134.62) (end 115.062 134.62) (width 0.45) (layer F.Cu) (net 22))
 (segment (start 121.158 115.638854) (end 121.881852 114.915002) (width 0.45) (layer F.Cu) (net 22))
 (segment (start 121.158 128.524) (end 121.158 115.638854) (width 0.45) (layer F.Cu) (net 22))
 (segment (start 115.062 134.62) (end 121.158 128.524) (width 0.45) (layer F.Cu) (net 22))
 (segment (start 134.62 134.62) (end 131.318 134.62) (width 0.45) (layer F.Cu) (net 23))
 (segment (start 125.222 115.638854) (end 124.498148 114.915002) (width 0.45) (layer F.Cu) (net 23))
 (segment (start 125.222 128.524) (end 125.222 115.638854) (width 0.45) (layer F.Cu) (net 23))
 (segment (start 131.318 134.62) (end 125.222 128.524) (width 0.45) (layer F.Cu) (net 23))
 (segment (start 134.62 132.08) (end 131.318 132.08) (width 0.45) (layer F.Cu) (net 24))
 (segment (start 126.238 115.523483) (end 125.063833 114.349316) (width 0.45) (layer F.Cu) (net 24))
 (segment (start 126.238 127) (end 126.238 115.523483) (width 0.45) (layer F.Cu) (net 24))
 (segment (start 131.318 132.08) (end 126.238 127) (width 0.45) (layer F.Cu) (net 24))
 (segment (start 134.62 129.54) (end 131.318 129.54) (width 0.45) (layer F.Cu) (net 25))
 (segment (start 127.254 115.408113) (end 125.629518 113.783631) (width 0.45) (layer F.Cu) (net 25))
 (segment (start 127.254 125.476) (end 127.254 115.408113) (width 0.45) (layer F.Cu) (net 25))
 (segment (start 131.318 129.54) (end 127.254 125.476) (width 0.45) (layer F.Cu) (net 25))
 (segment (start 134.62 127) (end 131.318 127) (width 0.45) (layer F.Cu) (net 26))
 (segment (start 128.27 115.292742) (end 126.195204 113.217946) (width 0.45) (layer F.Cu) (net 26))
 (segment (start 128.27 123.952) (end 128.27 115.292742) (width 0.45) (layer F.Cu) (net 26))
 (segment (start 131.318 127) (end 128.27 123.952) (width 0.45) (layer F.Cu) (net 26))
 (segment (start 134.62 124.46) (end 131.318 124.46) (width 0.45) (layer F.Cu) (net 27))
 (segment (start 129.286 115.177371) (end 126.760889 112.65226) (width 0.45) (layer F.Cu) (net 27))
 (segment (start 129.286 122.428) (end 129.286 115.177371) (width 0.45) (layer F.Cu) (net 27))
 (segment (start 131.318 124.46) (end 129.286 122.428) (width 0.45) (layer F.Cu) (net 27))
 (segment (start 134.62 121.92) (end 132.146 121.92) (width 0.45) (layer F.Cu) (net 28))
 (segment (start 132.146 121.92) (end 131.826 121.6) (width 0.45) (layer F.Cu) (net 28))
 (segment (start 131.826 121.6) (end 130.744 121.6) (width 0.45) (layer F.Cu) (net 28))
 (segment (start 130.744 121.6) (end 130.302 121.158) (width 0.45) (layer F.Cu) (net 28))
 (segment (start 130.302 121.158) (end 130.302 115.062) (width 0.45) (layer F.Cu) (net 28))
 (segment (start 130.302 115.062) (end 127.326575 112.086575) (width 0.45) (layer F.Cu) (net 28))
 (segment (start 131.826 119.7) (end 131.826 118.618) (width 0.45) (layer F.Cu) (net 29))
 (segment (start 131.826 118.618) (end 131.318 118.11) (width 0.45) (layer F.Cu) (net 29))
 (segment (start 131.318 118.11) (end 131.318 114.946629) (width 0.45) (layer F.Cu) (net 29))
 (segment (start 131.318 114.946629) (end 127.89226 111.520889) (width 0.45) (layer F.Cu) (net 29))
 (segment (start 134.62 119.38) (end 132.146 119.38) (width 0.45) (layer F.Cu) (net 29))
 (segment (start 132.146 119.38) (end 131.826 119.7) (width 0.45) (layer F.Cu) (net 29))
 (segment (start 134.62 116.84) (end 133.096 116.84) (width 0.45) (layer F.Cu) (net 30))
 (segment (start 132.334 114.831258) (end 128.457946 110.955204) (width 0.45) (layer F.Cu) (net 30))
 (segment (start 132.334 116.078) (end 132.334 114.831258) (width 0.45) (layer F.Cu) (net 30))
 (segment (start 133.096 116.84) (end 132.334 116.078) (width 0.45) (layer F.Cu) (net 30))
 (segment (start 134.62 114.3) (end 132.842 114.3) (width 0.45) (layer F.Cu) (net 31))
 (segment (start 132.842 114.3) (end 129.023631 110.481631) (width 0.45) (layer F.Cu) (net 31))
 (segment (start 129.023631 110.481631) (end 129.023631 110.389518) (width 0.45) (layer F.Cu) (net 31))
 (segment (start 134.62 111.76) (end 131.525483 111.76) (width 0.45) (layer F.Cu) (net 32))
 (segment (start 131.525483 111.76) (end 129.589316 109.823833) (width 0.45) (layer F.Cu) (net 32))
 (segment (start 134.62 109.22) (end 132.588 109.22) (width 0.45) (layer F.Cu) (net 33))
 (segment (start 130.878854 109.982) (end 130.155002 109.258148) (width 0.45) (layer F.Cu) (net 33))
 (segment (start 131.826 109.982) (end 130.878854 109.982) (width 0.45) (layer F.Cu) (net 33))
 (segment (start 132.588 109.22) (end 131.826 109.982) (width 0.45) (layer F.Cu) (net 33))
 (segment (start 134.62 106.68) (end 132.588 106.68) (width 0.45) (layer F.Cu) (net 34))
 (segment (start 130.878854 105.918) (end 130.155002 106.641852) (width 0.45) (layer F.Cu) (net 34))
 (segment (start 131.826 105.918) (end 130.878854 105.918) (width 0.45) (layer F.Cu) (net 34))
 (segment (start 132.588 106.68) (end 131.826 105.918) (width 0.45) (layer F.Cu) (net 34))
 (segment (start 134.62 104.14) (end 131.525483 104.14) (width 0.45) (layer F.Cu) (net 35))
 (segment (start 131.525483 104.14) (end 129.589316 106.076167) (width 0.45) (layer F.Cu) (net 35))
 (segment (start 134.62 101.6) (end 132.934113 101.6) (width 0.45) (layer F.Cu) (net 36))
 (segment (start 132.934113 101.6) (end 129.023631 105.510482) (width 0.45) (layer F.Cu) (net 36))
 (segment (start 134.62 99.06) (end 133.096 99.06) (width 0.45) (layer F.Cu) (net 37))
 (segment (start 132.334 101.068742) (end 128.457946 104.944796) (width 0.45) (layer F.Cu) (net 37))
 (segment (start 132.334 99.822) (end 132.334 101.068742) (width 0.45) (layer F.Cu) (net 37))
 (segment (start 133.096 99.06) (end 132.334 99.822) (width 0.45) (layer F.Cu) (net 37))
 (segment (start 134.62 96.52) (end 132.08 96.52) (width 0.45) (layer F.Cu) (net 38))
 (segment (start 131.318 100.953371) (end 127.89226 104.379111) (width 0.45) (layer F.Cu) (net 38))
 (segment (start 131.318 97.282) (end 131.318 100.953371) (width 0.45) (layer F.Cu) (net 38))
 (segment (start 132.08 96.52) (end 131.318 97.282) (width 0.45) (layer F.Cu) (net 38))
 (segment (start 134.62 93.98) (end 132.146 93.98) (width 0.45) (layer F.Cu) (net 39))
 (segment (start 132.146 93.98) (end 131.826 93.66) (width 0.45) (layer F.Cu) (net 39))
 (segment (start 131.826 93.66) (end 131.13 93.66) (width 0.45) (layer F.Cu) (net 39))
 (segment (start 131.13 93.66) (end 130.302 94.488) (width 0.45) (layer F.Cu) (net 39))
 (segment (start 130.302 94.488) (end 130.302 94.996) (width 0.45) (layer F.Cu) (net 39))
 (segment (start 130.302 100.838) (end 127.326575 103.813425) (width 0.45) (layer F.Cu) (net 39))
 (segment (start 130.302 94.996) (end 130.302 100.838) (width 0.45) (layer F.Cu) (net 39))
 (segment (start 134.62 91.44) (end 132.146 91.44) (width 0.45) (layer F.Cu) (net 40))
 (segment (start 132.146 91.44) (end 131.826 91.76) (width 0.45) (layer F.Cu) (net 40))
 (segment (start 131.826 91.76) (end 130.49 91.76) (width 0.45) (layer F.Cu) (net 40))
 (segment (start 130.49 91.76) (end 129.286 92.964) (width 0.45) (layer F.Cu) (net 40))
 (segment (start 129.286 100.722629) (end 126.760889 103.24774) (width 0.45) (layer F.Cu) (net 40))
 (segment (start 129.286 92.964) (end 129.286 100.722629) (width 0.45) (layer F.Cu) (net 40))
 (segment (start 134.62 88.9) (end 131.445 88.9) (width 0.45) (layer F.Cu) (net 41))
 (segment (start 128.27 100.607258) (end 126.195204 102.682054) (width 0.45) (layer F.Cu) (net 41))
 (segment (start 128.27 92.075) (end 128.27 100.607258) (width 0.45) (layer F.Cu) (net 41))
 (segment (start 131.445 88.9) (end 128.27 92.075) (width 0.45) (layer F.Cu) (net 41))
 (segment (start 134.62 86.36) (end 131.318 86.36) (width 0.45) (layer F.Cu) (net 42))
 (segment (start 127.254 100.491887) (end 125.629518 102.116369) (width 0.45) (layer F.Cu) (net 42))
 (segment (start 127.254 90.424) (end 127.254 100.491887) (width 0.45) (layer F.Cu) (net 42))
 (segment (start 131.318 86.36) (end 127.254 90.424) (width 0.45) (layer F.Cu) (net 42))
 (segment (start 134.62 83.82) (end 131.318 83.82) (width 0.45) (layer F.Cu) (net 43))
 (segment (start 126.238 100.376517) (end 125.063833 101.550684) (width 0.45) (layer F.Cu) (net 43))
 (segment (start 126.238 88.9) (end 126.238 100.376517) (width 0.45) (layer F.Cu) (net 43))
 (segment (start 131.318 83.82) (end 126.238 88.9) (width 0.45) (layer F.Cu) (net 43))
 (segment (start 125.233099 100.076486) (end 125.222 100.33) (width 0.45) (layer F.Cu) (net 44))
 (segment (start 125.222217 87.375783) (end 125.233099 100.076486) (width 0.45) (layer F.Cu) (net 44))
 (segment (start 125.222 100.33) (end 124.498148 100.984998) (width 0.45) (layer F.Cu) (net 44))
 (segment (start 131.318 81.28) (end 125.222217 87.375783) (width 0.45) (layer F.Cu) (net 44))
 (segment (start 134.62 81.28) (end 131.318 81.28) (width 0.45) (layer F.Cu) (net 44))
 (segment (start 116.924 117.602) (end 116.924 115.347371) (width 0.45) (layer F.Cu) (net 45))
 (segment (start 116.924 115.347371) (end 119.619111 112.65226) (width 0.45) (layer F.Cu) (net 45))
 (segment (start 116.586 122.09) (end 116.586 117.94) (width 0.45) (layer F.Cu) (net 45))
 (segment (start 116.586 117.94) (end 116.924 117.602) (width 0.45) (layer F.Cu) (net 45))
 (segment (start 111.76 73.914) (end 119.888 73.914) (width 0.45) (layer F.Cu) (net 46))
 (segment (start 122.682 76.708) (end 122.682 82.804) (width 0.45) (layer F.Cu) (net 46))
 (segment (start 119.888 73.914) (end 122.682 76.708) (width 0.45) (layer F.Cu) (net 46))
 (segment (start 134.62 76.454) (end 133.604 76.454) (width 0.45) (layer F.Cu) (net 47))
 (segment (start 133.604 76.454) (end 132.334 75.184) (width 0.45) (layer F.Cu) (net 47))
 (segment (start 132.334 75.184) (end 127.508 75.184) (width 0.45) (layer F.Cu) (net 47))
 (segment (start 127.508 75.184) (end 125.222 77.47) (width 0.45) (layer F.Cu) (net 47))
 (segment (start 125.222 77.47) (end 125.222 82.804) (width 0.45) (layer F.Cu) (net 47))
 (segment (start 123.19 88.646) (end 123.19 87.376) (width 0.45) (layer F.Cu) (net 49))
 (segment (start 127.254 81.026) (end 126.492 80.264) (width 0.45) (layer F.Cu) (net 49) (status 800000))
 (segment (start 127.254 83.312) (end 127.254 81.026) (width 0.45) (layer F.Cu) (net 49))
 (segment (start 126.492 84.074) (end 127.254 83.312) (width 0.45) (layer F.Cu) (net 49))
 (segment (start 123.19 87.376) (end 126.492 84.074) (width 0.45) (layer F.Cu) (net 49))
 (segment (start 134.62 73.914) (end 126.746 73.914) (width 0.45) (layer F.Cu) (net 50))
 (segment (start 123.952 76.708) (end 123.952 80.264) (width 0.45) (layer F.Cu) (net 50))
 (segment (start 126.746 73.914) (end 123.952 76.708) (width 0.45) (layer F.Cu) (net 50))
 (segment (start 111.76 76.454) (end 113.538 76.454) (width 0.45) (layer F.Cu) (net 51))
 (segment (start 121.412 77.47) (end 121.412 80.264) (width 0.45) (layer F.Cu) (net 51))
 (segment (start 119.126 75.184) (end 121.412 77.47) (width 0.45) (layer F.Cu) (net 51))
 (segment (start 114.808 75.184) (end 119.126 75.184) (width 0.45) (layer F.Cu) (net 51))
 (segment (start 113.538 76.454) (end 114.808 75.184) (width 0.45) (layer F.Cu) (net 51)))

